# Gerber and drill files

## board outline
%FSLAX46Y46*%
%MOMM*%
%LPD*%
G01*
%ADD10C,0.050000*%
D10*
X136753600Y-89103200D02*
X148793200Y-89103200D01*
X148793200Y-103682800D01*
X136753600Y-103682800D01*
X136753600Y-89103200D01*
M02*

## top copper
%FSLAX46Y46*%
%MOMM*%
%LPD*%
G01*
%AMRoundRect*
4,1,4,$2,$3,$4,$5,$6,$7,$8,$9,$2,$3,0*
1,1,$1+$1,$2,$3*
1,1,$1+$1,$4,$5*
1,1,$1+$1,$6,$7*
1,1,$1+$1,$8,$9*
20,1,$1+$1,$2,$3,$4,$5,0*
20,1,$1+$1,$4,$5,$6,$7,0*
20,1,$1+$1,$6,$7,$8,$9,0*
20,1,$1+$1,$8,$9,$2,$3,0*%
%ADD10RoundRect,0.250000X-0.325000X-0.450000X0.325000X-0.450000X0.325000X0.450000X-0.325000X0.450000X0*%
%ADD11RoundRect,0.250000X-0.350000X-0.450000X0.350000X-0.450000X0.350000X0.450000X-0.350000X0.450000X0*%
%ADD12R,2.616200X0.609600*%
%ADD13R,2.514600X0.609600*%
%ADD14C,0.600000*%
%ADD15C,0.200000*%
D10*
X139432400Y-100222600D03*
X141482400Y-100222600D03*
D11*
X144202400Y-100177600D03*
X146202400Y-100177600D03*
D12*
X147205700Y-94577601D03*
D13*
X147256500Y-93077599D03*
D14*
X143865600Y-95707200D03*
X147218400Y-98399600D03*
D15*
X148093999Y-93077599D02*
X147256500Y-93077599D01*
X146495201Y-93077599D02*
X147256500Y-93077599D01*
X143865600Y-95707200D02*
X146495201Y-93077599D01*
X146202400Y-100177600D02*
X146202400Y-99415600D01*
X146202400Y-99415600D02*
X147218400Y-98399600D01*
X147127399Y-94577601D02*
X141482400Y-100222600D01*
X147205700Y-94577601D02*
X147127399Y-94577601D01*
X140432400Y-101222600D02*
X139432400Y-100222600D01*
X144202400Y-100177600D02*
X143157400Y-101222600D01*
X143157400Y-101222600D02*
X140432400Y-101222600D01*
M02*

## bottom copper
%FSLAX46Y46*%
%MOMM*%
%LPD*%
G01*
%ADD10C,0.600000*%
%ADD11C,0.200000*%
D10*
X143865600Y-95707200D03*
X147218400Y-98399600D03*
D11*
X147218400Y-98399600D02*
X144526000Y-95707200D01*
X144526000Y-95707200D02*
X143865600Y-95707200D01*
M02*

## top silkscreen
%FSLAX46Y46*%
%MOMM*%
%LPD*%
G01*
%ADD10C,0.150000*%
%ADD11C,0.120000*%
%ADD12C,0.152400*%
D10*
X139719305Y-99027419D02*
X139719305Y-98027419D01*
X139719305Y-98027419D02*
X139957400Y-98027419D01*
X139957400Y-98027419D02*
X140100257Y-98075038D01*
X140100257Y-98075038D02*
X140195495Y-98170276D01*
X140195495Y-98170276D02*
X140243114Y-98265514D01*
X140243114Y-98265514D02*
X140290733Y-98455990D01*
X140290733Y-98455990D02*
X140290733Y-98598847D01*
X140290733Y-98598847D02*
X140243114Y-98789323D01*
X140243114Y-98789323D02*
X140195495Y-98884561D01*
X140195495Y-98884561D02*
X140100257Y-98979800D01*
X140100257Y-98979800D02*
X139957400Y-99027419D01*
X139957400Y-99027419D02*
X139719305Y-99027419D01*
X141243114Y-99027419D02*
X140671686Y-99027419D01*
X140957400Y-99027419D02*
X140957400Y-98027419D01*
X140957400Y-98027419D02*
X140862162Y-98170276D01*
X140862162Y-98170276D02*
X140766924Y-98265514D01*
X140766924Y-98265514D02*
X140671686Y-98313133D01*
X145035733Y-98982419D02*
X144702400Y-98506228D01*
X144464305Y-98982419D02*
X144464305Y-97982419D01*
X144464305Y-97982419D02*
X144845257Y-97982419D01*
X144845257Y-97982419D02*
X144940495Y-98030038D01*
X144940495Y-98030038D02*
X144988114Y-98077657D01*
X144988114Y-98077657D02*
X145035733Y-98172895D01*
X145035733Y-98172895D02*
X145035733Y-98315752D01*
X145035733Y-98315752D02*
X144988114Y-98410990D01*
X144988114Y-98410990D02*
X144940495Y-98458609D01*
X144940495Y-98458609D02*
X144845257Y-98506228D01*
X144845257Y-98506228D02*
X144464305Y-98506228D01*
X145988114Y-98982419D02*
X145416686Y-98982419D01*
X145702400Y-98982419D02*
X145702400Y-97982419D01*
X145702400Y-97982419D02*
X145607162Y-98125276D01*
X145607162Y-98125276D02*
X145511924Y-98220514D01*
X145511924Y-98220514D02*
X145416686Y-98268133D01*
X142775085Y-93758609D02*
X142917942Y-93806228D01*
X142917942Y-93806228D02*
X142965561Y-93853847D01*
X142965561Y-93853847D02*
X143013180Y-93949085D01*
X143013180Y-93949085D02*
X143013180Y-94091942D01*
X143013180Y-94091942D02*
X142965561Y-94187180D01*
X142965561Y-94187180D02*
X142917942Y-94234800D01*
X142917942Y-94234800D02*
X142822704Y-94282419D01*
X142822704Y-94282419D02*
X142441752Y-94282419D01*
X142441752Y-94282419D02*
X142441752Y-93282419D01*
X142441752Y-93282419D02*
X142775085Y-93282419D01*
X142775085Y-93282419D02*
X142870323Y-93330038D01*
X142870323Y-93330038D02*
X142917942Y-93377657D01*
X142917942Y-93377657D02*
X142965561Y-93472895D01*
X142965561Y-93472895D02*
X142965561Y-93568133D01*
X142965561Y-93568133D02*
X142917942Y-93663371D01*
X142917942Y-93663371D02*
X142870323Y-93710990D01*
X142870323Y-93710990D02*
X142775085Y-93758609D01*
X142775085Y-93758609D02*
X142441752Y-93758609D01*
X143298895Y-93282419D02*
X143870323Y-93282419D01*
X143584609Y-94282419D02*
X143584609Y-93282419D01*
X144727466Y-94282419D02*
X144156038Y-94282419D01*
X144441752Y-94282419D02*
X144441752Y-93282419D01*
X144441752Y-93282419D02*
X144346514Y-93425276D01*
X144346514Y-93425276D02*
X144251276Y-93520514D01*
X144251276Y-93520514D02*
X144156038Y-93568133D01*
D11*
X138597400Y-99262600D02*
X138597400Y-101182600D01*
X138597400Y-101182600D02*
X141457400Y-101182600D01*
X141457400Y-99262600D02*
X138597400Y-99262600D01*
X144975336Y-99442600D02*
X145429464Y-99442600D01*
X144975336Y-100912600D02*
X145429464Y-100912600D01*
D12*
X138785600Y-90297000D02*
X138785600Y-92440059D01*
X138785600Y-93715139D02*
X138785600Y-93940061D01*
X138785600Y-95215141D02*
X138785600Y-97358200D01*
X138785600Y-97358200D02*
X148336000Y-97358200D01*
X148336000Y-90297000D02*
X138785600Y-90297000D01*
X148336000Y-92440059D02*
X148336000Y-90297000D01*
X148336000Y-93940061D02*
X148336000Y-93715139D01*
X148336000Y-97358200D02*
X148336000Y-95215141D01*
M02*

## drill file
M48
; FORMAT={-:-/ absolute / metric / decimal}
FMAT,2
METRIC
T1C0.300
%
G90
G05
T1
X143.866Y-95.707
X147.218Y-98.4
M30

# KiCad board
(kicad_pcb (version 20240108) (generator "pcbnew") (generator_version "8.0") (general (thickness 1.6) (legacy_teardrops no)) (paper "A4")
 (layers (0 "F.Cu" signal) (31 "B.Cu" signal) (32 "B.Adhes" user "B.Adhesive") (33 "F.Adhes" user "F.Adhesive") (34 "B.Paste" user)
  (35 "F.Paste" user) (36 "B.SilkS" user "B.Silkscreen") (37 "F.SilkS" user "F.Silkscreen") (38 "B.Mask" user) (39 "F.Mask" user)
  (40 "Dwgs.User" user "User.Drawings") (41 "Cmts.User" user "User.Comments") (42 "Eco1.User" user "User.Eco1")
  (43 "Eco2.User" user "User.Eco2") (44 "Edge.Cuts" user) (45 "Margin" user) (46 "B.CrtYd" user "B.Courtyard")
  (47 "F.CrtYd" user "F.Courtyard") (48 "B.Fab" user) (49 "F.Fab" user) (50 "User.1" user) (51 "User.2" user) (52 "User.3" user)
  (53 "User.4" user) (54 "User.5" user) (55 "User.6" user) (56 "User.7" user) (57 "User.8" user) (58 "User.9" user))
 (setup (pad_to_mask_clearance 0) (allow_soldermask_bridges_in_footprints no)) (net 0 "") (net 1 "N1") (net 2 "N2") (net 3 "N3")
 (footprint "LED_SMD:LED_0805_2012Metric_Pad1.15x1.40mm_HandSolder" (layer "F.Cu") (at 140.4574 100.2226)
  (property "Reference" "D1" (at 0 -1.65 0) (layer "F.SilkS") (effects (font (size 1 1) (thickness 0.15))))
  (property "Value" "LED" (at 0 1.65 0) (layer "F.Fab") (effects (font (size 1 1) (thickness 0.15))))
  (fp_line (start -1.86 -0.96) (end -1.86 0.96) (stroke (width 0.12) (type solid)) (layer "F.SilkS"))
  (fp_line (start -1.86 0.96) (end 1 0.96) (stroke (width 0.12) (type solid)) (layer "F.SilkS"))
  (fp_line (start 1 -0.96) (end -1.86 -0.96) (stroke (width 0.12) (type solid)) (layer "F.SilkS"))
  (pad "1" smd roundrect (at -1.025 0) (size 1.15 1.4) (layers "F.Cu" "F.Paste" "F.Mask") (roundrect_rratio 0.217391) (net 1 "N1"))
  (pad "2" smd roundrect (at 1.025 0) (size 1.15 1.4) (layers "F.Cu" "F.Paste" "F.Mask") (roundrect_rratio 0.217391) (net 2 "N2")))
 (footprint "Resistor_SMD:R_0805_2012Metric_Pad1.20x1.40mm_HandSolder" (layer "F.Cu") (at 145.2024 100.1776)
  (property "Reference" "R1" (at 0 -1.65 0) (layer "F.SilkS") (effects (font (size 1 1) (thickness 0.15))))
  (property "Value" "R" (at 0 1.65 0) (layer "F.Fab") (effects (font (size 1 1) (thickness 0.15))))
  (fp_line (start -0.227064 -0.735) (end 0.227064 -0.735) (stroke (width 0.12) (type solid)) (layer "F.SilkS"))
  (fp_line (start -0.227064 0.735) (end 0.227064 0.735) (stroke (width 0.12) (type solid)) (layer "F.SilkS"))
  (pad "1" smd roundrect (at -1 0) (size 1.2 1.4) (layers "F.Cu" "F.Paste" "F.Mask") (roundrect_rratio 0.208333) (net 1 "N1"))
  (pad "2" smd roundrect (at 1 0) (size 1.2 1.4) (layers "F.Cu" "F.Paste" "F.Mask") (roundrect_rratio 0.208333) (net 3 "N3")))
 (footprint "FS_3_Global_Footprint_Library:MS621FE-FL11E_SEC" (layer "F.Cu") (at 143.5608 93.8276 180)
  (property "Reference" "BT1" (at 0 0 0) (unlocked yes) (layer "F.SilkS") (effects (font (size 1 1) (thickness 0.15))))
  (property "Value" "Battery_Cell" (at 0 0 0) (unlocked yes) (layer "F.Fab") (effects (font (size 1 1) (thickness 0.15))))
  (fp_line (start 4.7752 3.5306) (end 4.7752 1.387541) (stroke (width 0.1524) (type solid)) (layer "F.SilkS"))
  (fp_line (start 4.7752 0.112461) (end 4.7752 -0.112461) (stroke (width 0.1524) (type solid)) (layer "F.SilkS"))
  (fp_line (start 4.7752 -1.387541) (end 4.7752 -3.5306) (stroke (width 0.1524) (type solid)) (layer "F.SilkS"))
  (fp_line (start 4.7752 -3.5306) (end -4.7752 -3.5306) (stroke (width 0.1524) (type solid)) (layer "F.SilkS"))
  (fp_line (start -4.7752 3.5306) (end 4.7752 3.5306) (stroke (width 0.1524) (type solid)) (layer "F.SilkS"))
  (fp_line (start -4.7752 1.387541) (end -4.7752 3.5306) (stroke (width 0.1524) (type solid)) (layer "F.SilkS"))
  (fp_line (start -4.7752 -0.112461) (end -4.7752 0.112461) (stroke (width 0.1524) (type solid)) (layer "F.SilkS"))
  (fp_line (start -4.7752 -3.5306) (end -4.7752 -1.387541) (stroke (width 0.1524) (type solid)) (layer "F.SilkS"))
  (pad "1" smd rect (at -3.6449 -0.750001 180) (size 2.6162 0.6096) (layers "F.Cu" "F.Paste" "F.Mask") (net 2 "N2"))
  (pad "2" smd rect (at -3.6957 0.750001 180) (size 2.5146 0.6096) (layers "F.Cu" "F.Paste" "F.Mask") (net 3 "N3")))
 (gr_rect (start 136.7536 89.1032) (end 148.7932 103.6828) (stroke (width 0.05) (type default)) (fill none) (layer "Edge.Cuts"))
 (segment (start 148.093999 93.077599) (end 147.2565 93.077599) (width 0.2) (layer "F.Cu") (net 3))
 (segment (start 146.495201 93.077599) (end 147.2565 93.077599) (width 0.2) (layer "F.Cu") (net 3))
 (segment (start 143.8656 95.7072) (end 146.495201 93.077599) (width 0.2) (layer "F.Cu") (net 3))
 (segment (start 146.2024 100.1776) (end 146.2024 99.4156) (width 0.2) (layer "F.Cu") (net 3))
 (segment (start 146.2024 99.4156) (end 147.2184 98.3996) (width 0.2) (layer "F.Cu") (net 3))
 (via (at 143.8656 95.7072) (size 0.6) (drill 0.3) (layers "F.Cu" "B.Cu") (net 3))
 (via (at 147.2184 98.3996) (size 0.6) (drill 0.3) (layers "F.Cu" "B.Cu") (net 3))
 (segment (start 147.2184 98.3996) (end 144.526 95.7072) (width 0.2) (layer "B.Cu") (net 3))
 (segment (start 144.526 95.7072) (end 143.8656 95.7072) (width 0.2) (layer "B.Cu") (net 3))
 (segment (start 147.127399 94.577601) (end 141.4824 100.2226) (width 0.2) (layer "F.Cu") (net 2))
 (segment (start 147.2057 94.577601) (end 147.127399 94.577601) (width 0.2) (layer "F.Cu") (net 2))
 (segment (start 140.4324 101.2226) (end 139.4324 100.2226) (width 0.2) (layer "F.Cu") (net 1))
 (segment (start 144.2024 100.1776) (end 143.1574 101.2226) (width 0.2) (layer "F.Cu") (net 1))
 (segment (start 143.1574 101.2226) (end 140.4324 101.2226) (width 0.2) (layer "F.Cu") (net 1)))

